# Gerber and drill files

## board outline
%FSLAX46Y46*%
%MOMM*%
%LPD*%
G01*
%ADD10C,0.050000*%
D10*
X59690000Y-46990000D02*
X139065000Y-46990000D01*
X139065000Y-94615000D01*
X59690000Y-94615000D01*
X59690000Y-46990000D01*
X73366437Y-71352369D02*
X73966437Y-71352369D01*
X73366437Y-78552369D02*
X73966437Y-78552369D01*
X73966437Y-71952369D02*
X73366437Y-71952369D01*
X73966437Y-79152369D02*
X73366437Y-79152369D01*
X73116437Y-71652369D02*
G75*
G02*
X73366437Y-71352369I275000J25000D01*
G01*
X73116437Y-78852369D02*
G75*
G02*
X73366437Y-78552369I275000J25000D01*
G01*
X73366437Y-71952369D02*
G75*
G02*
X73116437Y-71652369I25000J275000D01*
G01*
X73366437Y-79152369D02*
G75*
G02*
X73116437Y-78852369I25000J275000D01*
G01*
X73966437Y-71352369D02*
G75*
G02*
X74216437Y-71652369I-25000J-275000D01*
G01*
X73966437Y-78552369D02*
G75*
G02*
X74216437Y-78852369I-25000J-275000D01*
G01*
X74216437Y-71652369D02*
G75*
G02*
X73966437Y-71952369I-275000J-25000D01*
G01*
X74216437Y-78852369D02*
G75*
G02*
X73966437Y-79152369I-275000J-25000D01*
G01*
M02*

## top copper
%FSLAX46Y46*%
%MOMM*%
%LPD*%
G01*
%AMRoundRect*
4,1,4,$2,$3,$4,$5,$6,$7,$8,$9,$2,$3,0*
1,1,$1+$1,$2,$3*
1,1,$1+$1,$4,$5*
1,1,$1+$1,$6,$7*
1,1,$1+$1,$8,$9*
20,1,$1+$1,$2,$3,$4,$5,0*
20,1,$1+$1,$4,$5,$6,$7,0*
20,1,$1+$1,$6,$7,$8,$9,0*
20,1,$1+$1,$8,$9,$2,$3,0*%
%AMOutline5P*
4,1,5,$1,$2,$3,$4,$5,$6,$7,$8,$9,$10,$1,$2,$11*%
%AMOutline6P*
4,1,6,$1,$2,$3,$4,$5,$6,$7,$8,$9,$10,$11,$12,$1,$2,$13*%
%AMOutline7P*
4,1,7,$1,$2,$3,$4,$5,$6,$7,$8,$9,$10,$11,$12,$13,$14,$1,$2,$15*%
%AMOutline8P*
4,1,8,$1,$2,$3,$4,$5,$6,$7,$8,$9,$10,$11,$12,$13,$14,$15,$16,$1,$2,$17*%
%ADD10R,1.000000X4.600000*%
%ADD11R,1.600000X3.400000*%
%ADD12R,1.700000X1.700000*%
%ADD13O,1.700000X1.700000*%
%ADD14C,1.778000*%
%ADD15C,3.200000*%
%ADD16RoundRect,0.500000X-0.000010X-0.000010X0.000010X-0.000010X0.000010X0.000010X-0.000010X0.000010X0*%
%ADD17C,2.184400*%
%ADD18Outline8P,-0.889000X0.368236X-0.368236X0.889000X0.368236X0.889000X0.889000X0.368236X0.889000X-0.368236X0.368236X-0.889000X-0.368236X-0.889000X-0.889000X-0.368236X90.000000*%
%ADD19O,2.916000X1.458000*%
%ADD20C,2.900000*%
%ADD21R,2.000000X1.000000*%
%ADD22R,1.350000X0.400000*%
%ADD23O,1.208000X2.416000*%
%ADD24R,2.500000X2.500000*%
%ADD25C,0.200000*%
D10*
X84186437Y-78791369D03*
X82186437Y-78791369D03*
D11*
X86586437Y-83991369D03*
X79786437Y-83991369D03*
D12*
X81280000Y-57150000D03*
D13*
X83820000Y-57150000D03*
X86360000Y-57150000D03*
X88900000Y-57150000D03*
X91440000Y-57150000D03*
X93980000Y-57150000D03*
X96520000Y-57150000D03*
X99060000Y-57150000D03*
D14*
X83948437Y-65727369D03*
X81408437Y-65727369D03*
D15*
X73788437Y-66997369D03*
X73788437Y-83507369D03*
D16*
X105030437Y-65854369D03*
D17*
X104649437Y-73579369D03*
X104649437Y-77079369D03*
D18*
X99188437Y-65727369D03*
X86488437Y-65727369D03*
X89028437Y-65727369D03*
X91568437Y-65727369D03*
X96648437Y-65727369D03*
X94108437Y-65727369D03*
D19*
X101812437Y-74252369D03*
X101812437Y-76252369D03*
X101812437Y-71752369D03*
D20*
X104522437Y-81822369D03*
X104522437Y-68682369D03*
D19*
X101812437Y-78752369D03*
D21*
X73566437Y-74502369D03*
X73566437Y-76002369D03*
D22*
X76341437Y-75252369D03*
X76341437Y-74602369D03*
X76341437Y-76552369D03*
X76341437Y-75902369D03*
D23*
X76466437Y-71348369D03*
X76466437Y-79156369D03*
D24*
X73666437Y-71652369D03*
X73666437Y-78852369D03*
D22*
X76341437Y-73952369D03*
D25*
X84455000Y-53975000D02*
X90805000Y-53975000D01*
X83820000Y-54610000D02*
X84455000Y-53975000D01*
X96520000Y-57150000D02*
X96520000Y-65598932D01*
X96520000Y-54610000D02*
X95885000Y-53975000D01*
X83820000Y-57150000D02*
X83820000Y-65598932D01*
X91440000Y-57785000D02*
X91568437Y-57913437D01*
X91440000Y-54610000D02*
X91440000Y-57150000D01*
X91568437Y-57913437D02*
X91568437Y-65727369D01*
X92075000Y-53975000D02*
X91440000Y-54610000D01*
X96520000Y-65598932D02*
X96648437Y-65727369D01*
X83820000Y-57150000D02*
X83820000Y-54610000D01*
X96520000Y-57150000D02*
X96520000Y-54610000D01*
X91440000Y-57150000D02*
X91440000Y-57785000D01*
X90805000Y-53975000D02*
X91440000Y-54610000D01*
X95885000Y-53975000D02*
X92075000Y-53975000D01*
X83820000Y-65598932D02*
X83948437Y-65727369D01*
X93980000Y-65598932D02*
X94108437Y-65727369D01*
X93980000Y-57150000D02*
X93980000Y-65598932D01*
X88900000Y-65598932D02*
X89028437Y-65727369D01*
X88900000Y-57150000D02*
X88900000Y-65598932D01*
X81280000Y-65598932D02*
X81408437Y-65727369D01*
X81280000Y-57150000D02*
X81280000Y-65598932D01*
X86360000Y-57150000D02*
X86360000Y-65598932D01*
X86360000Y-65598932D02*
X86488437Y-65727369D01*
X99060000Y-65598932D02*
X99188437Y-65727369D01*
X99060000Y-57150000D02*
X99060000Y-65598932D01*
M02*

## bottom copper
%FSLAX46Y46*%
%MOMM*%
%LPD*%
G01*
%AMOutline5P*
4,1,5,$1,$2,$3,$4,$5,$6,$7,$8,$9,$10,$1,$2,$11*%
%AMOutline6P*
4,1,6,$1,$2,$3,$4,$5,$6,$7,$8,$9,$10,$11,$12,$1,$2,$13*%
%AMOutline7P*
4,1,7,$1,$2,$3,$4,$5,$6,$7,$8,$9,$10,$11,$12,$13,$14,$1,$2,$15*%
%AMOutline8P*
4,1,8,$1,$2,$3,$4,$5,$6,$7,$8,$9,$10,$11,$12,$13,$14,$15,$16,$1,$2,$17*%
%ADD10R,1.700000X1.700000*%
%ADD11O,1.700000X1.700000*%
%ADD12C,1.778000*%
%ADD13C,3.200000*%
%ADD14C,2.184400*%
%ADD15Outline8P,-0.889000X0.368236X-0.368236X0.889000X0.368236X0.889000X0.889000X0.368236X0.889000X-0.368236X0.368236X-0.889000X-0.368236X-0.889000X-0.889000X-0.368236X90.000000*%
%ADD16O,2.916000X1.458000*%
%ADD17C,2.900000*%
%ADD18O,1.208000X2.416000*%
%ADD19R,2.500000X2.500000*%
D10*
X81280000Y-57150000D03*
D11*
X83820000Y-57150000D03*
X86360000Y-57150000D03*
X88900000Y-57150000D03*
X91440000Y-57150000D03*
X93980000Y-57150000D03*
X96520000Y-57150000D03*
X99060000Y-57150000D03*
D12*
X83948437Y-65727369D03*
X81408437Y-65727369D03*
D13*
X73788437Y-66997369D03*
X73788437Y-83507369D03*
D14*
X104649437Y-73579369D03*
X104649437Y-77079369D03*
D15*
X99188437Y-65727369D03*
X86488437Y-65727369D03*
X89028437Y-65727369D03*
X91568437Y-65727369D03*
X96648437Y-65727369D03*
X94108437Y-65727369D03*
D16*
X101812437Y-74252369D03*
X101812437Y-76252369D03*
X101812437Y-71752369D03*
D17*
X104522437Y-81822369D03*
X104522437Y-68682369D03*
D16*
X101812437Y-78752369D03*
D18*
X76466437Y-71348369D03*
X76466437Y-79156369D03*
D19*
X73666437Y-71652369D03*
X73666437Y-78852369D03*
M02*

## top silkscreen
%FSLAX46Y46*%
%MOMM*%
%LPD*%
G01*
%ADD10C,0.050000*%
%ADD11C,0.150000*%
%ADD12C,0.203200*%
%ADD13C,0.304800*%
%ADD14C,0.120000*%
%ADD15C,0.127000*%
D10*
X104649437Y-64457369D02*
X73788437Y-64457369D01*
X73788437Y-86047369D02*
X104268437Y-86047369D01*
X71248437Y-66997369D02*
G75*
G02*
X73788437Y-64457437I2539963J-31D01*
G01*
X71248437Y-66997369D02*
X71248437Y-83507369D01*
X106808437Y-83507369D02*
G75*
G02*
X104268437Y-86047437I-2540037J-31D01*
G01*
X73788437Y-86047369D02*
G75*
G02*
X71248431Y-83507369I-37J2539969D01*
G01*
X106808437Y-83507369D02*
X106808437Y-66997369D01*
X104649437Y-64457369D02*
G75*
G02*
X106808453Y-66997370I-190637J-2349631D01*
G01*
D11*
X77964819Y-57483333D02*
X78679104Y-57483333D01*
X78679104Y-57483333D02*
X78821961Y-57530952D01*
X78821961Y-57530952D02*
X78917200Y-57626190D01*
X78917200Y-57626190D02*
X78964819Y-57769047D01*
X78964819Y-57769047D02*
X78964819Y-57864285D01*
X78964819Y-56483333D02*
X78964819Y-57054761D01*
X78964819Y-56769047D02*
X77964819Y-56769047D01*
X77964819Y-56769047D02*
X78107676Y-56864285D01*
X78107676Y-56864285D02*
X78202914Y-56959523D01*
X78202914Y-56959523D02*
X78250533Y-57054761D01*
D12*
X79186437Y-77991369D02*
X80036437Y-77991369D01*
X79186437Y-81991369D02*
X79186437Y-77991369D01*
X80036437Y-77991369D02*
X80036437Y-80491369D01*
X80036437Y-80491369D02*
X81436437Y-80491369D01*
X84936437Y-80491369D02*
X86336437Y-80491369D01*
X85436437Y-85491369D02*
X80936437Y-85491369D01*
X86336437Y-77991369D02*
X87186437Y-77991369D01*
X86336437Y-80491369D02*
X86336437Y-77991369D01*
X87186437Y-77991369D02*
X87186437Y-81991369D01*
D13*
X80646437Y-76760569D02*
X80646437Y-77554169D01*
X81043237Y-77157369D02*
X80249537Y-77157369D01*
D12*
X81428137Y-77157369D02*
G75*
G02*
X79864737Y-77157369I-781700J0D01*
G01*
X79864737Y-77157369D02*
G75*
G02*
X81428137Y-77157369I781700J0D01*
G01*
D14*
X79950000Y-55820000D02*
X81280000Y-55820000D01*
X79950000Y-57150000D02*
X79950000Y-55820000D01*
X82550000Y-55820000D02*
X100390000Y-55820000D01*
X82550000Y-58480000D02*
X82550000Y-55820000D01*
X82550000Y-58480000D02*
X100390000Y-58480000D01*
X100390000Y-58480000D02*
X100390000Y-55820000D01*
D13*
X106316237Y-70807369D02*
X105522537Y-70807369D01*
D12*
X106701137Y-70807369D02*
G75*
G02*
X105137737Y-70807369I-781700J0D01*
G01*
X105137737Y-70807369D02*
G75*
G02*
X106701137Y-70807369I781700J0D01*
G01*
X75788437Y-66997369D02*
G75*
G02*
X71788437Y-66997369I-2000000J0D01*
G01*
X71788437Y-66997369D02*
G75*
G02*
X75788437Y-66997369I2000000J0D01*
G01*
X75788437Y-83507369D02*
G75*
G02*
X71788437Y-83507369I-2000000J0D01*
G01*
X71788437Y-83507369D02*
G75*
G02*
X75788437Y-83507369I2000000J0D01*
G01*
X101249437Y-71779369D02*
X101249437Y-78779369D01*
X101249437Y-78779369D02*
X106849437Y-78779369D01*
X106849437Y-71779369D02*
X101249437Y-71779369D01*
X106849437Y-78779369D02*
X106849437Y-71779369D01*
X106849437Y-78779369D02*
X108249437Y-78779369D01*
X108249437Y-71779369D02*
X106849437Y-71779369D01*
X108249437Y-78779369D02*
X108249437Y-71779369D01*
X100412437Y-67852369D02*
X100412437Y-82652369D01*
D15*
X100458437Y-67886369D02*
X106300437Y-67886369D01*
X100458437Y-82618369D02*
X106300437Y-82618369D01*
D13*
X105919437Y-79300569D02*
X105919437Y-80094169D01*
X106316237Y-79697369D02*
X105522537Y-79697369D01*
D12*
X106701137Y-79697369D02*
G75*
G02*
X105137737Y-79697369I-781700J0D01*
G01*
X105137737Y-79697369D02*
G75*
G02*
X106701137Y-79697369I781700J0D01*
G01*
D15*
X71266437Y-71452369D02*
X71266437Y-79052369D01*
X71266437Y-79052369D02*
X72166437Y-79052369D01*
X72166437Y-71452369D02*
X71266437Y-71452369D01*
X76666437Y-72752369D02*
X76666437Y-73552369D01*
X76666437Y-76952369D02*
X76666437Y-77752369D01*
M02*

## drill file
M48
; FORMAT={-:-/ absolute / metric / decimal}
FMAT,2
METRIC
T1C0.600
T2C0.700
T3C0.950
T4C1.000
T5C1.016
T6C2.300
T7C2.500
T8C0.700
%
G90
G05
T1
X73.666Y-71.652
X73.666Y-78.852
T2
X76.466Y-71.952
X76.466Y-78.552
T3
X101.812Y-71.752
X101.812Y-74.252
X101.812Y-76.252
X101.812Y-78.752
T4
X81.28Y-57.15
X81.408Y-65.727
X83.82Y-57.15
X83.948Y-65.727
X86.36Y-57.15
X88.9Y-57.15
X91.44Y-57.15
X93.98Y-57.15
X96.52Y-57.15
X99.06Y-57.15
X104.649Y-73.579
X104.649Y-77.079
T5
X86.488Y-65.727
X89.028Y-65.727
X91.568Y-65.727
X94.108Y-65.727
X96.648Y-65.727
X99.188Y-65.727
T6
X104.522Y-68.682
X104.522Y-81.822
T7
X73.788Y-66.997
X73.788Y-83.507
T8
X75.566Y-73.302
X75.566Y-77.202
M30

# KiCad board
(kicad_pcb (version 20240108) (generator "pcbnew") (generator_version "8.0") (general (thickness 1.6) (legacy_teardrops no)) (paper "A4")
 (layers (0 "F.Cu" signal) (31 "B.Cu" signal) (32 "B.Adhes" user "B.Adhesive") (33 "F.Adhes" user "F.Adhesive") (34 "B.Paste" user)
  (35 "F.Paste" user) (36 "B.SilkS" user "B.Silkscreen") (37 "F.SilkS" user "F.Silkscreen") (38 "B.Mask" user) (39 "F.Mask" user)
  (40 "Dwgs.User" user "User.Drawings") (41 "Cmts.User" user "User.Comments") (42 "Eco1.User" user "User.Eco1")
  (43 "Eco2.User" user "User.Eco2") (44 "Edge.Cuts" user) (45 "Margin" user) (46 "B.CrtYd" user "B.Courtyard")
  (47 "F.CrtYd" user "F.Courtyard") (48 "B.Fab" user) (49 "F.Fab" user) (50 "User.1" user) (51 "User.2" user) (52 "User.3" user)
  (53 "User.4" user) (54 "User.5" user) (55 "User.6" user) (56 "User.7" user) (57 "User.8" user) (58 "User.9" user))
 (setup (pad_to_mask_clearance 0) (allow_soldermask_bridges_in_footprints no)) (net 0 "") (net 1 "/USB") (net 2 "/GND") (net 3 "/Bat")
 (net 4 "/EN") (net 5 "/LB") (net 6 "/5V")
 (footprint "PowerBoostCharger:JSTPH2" (layer "F.Cu") (at 83.186437 82.491369 180)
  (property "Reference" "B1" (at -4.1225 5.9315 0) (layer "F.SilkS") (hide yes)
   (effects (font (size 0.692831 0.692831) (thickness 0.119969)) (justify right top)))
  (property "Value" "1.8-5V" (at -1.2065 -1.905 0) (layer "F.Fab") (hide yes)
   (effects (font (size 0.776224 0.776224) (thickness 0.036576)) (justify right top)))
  (fp_line (start 4 4.5) (end 3.15 4.5) (stroke (width 0.2032) (type solid)) (layer "F.SilkS"))
  (fp_line (start 4 0.5) (end 4 4.5) (stroke (width 0.2032) (type solid)) (layer "F.SilkS"))
  (fp_line (start 3.15 4.5) (end 3.15 2) (stroke (width 0.2032) (type solid)) (layer "F.SilkS"))
  (fp_line (start 3.15 2) (end 1.75 2) (stroke (width 0.2032) (type solid)) (layer "F.SilkS"))
  (fp_line (start -1.75 2) (end -3.15 2) (stroke (width 0.2032) (type solid)) (layer "F.SilkS"))
  (fp_line (start -2.25 -3) (end 2.25 -3) (stroke (width 0.2032) (type solid)) (layer "F.SilkS"))
  (fp_line (start -3.15 4.5) (end -4 4.5) (stroke (width 0.2032) (type solid)) (layer "F.SilkS"))
  (fp_line (start -3.15 2) (end -3.15 4.5) (stroke (width 0.2032) (type solid)) (layer "F.SilkS"))
  (fp_line (start -4 4.5) (end -4 0.5) (stroke (width 0.2032) (type solid)) (layer "F.SilkS"))
  (pad "1" smd rect (at -1 3.7 180) (size 1 4.6) (layers "F.Cu" "F.Paste" "F.Mask") (solder_mask_margin 0.0508) (thermal_bridge_angle 45))
  (pad "2" smd rect (at 1 3.7 180) (size 1 4.6) (layers "F.Cu" "F.Paste" "F.Mask") (solder_mask_margin 0.0508) (thermal_bridge_angle 45))
  (pad "NC1" smd rect (at -3.4 -1.5 270) (size 3.4 1.6) (layers "F.Cu" "F.Paste" "F.Mask") (solder_mask_margin 0.0508)
   (thermal_bridge_angle 45))
  (pad "NC2" smd rect (at 3.4 -1.5 270) (size 3.4 1.6) (layers "F.Cu" "F.Paste" "F.Mask") (solder_mask_margin 0.0508)
   (thermal_bridge_angle 45)))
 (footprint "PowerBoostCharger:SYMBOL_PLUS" (layer "F.Cu") (at 80.646437 77.157369)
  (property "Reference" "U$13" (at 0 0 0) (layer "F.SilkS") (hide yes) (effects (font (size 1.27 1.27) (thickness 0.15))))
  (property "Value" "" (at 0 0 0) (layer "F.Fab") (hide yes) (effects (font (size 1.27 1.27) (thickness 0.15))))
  (fp_line (start 0 -0.3968) (end 0 0.3968) (stroke (width 0.3048) (type solid)) (layer "F.SilkS"))
  (fp_line (start 0.3968 0) (end -0.3969 0) (stroke (width 0.3048) (type solid)) (layer "F.SilkS"))
  (fp_circle (center 0 0) (end 0.7817 0) (stroke (width 0.2032) (type solid)) (fill none) (layer "F.SilkS")))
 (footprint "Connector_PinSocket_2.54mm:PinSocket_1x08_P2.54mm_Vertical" (layer "F.Cu") (at 81.28 57.15 90)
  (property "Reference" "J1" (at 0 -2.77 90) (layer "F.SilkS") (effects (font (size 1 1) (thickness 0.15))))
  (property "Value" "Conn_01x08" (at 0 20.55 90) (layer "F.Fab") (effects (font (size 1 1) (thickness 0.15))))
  (fp_line (start 1.33 -1.33) (end 1.33 0) (stroke (width 0.12) (type solid)) (layer "F.SilkS"))
  (fp_line (start 0 -1.33) (end 1.33 -1.33) (stroke (width 0.12) (type solid)) (layer "F.SilkS"))
  (fp_line (start 1.33 1.27) (end 1.33 19.11) (stroke (width 0.12) (type solid)) (layer "F.SilkS"))
  (fp_line (start -1.33 1.27) (end 1.33 1.27) (stroke (width 0.12) (type solid)) (layer "F.SilkS"))
  (fp_line (start -1.33 1.27) (end -1.33 19.11) (stroke (width 0.12) (type solid)) (layer "F.SilkS"))
  (fp_line (start -1.33 19.11) (end 1.33 19.11) (stroke (width 0.12) (type solid)) (layer "F.SilkS"))
  (pad "1" thru_hole rect (at 0 0 90) (size 1.7 1.7) (drill 1) (layers "*.Cu" "*.Mask") (remove_unused_layers no) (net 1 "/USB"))
  (pad "2" thru_hole oval (at 0 2.54 90) (size 1.7 1.7) (drill 1) (layers "*.Cu" "*.Mask") (remove_unused_layers no) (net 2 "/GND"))
  (pad "3" thru_hole oval (at 0 5.08 90) (size 1.7 1.7) (drill 1) (layers "*.Cu" "*.Mask") (remove_unused_layers no) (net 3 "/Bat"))
  (pad "4" thru_hole oval (at 0 7.62 90) (size 1.7 1.7) (drill 1) (layers "*.Cu" "*.Mask") (remove_unused_layers no) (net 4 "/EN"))
  (pad "5" thru_hole oval (at 0 10.16 90) (size 1.7 1.7) (drill 1) (layers "*.Cu" "*.Mask") (remove_unused_layers no) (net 2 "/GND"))
  (pad "6" thru_hole oval (at 0 12.7 90) (size 1.7 1.7) (drill 1) (layers "*.Cu" "*.Mask") (remove_unused_layers no) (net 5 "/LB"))
  (pad "7" thru_hole oval (at 0 15.24 90) (size 1.7 1.7) (drill 1) (layers "*.Cu" "*.Mask") (remove_unused_layers no) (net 2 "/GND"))
  (pad "8" thru_hole oval (at 0 17.78 90) (size 1.7 1.7) (drill 1) (layers "*.Cu" "*.Mask") (remove_unused_layers no) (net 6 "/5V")))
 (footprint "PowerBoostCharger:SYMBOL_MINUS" (layer "F.Cu") (at 105.919437 70.807369)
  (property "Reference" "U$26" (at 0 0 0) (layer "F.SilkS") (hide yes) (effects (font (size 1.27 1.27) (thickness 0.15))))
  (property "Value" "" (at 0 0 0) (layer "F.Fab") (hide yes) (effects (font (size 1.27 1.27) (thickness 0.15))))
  (fp_line (start 0.3968 0) (end -0.3969 0) (stroke (width 0.3048) (type solid)) (layer "F.SilkS"))
  (fp_circle (center 0 0) (end 0.7817 0) (stroke (width 0.2032) (type solid)) (fill none) (layer "F.SilkS")))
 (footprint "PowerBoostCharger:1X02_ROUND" (layer "F.Cu") (at 82.678437 65.727369)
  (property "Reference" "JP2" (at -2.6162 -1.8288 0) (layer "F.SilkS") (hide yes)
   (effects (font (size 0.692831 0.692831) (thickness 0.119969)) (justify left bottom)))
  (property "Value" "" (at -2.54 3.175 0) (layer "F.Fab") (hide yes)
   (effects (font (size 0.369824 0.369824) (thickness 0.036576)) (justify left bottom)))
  (pad "GND" thru_hole circle (at 1.27 0 90) (size 1.778 1.778) (drill 1) (layers "*.Cu" "*.Mask") (remove_unused_layers no) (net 2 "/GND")
   (solder_mask_margin 0.0508))
  (pad "USB" thru_hole circle (at -1.27 0 90) (size 1.778 1.778) (drill 1) (layers "*.Cu" "*.Mask") (remove_unused_layers no) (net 1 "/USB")
   (solder_mask_margin 0.0508)))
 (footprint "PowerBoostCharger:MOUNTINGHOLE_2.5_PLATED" (layer "F.Cu") (at 73.788437 66.997369)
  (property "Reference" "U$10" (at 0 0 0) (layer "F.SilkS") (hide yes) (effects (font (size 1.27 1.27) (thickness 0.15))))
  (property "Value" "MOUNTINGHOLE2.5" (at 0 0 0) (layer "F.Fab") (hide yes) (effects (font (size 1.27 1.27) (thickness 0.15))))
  (fp_circle (center 0 0) (end 2 0) (stroke (width 0.2032) (type solid)) (fill none) (layer "F.SilkS"))
  (pad "P$1" thru_hole circle (at 0 0) (size 3.2 3.2) (drill 2.5) (layers "*.Cu" "*.Mask") (remove_unused_layers no)
   (solder_mask_margin 0.0508))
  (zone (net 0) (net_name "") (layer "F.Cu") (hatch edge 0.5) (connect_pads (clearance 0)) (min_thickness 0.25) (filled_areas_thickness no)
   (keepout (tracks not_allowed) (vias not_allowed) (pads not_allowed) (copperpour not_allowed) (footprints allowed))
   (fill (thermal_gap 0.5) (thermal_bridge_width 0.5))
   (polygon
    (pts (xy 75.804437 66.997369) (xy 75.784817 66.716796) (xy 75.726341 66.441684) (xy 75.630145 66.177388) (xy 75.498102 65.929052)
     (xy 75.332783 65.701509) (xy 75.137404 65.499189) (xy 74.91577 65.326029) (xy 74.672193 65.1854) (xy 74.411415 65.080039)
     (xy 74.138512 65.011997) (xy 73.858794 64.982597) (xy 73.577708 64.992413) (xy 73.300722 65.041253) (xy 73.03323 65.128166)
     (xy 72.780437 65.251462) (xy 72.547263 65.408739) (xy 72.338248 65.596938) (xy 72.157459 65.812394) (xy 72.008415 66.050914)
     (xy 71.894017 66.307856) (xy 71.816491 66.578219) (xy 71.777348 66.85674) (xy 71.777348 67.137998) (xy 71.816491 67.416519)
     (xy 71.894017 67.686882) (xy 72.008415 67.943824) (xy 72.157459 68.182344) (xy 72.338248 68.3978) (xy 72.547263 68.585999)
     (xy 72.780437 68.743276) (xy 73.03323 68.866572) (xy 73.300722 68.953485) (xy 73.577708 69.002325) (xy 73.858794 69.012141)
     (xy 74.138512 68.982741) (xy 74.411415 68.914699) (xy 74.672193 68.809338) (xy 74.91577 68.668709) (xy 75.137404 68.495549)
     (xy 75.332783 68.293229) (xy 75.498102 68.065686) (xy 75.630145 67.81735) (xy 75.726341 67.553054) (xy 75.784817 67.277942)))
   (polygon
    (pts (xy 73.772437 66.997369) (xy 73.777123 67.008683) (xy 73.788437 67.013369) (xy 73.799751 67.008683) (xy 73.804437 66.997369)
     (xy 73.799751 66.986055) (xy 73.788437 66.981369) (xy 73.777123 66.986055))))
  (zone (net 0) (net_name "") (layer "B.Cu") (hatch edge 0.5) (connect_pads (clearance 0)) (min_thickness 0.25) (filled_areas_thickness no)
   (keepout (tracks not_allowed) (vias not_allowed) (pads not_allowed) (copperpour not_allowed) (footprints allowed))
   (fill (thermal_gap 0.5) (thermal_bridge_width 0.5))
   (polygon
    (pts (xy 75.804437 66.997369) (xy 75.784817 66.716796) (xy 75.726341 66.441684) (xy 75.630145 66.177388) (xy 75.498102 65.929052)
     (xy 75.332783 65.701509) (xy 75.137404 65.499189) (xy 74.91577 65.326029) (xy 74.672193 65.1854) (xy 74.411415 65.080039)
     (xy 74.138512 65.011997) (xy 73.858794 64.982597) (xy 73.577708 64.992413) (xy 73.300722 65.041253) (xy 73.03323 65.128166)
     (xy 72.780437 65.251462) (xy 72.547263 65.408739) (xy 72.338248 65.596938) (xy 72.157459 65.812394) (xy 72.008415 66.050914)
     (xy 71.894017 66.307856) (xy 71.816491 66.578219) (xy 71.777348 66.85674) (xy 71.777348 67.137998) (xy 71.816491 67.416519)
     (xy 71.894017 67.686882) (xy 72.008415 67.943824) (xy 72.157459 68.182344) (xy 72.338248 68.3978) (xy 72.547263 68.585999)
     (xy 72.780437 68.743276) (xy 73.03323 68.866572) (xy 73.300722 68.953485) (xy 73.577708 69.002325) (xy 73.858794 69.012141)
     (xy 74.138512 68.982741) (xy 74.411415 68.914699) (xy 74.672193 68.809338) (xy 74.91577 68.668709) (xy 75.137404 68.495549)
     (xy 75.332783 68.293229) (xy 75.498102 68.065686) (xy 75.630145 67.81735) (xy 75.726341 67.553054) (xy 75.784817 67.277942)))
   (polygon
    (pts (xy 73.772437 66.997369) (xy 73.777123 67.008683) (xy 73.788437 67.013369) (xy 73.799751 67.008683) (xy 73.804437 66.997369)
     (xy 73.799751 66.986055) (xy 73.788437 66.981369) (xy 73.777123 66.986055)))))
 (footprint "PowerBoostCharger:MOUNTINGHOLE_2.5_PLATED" (layer "F.Cu") (at 73.788437 83.507369)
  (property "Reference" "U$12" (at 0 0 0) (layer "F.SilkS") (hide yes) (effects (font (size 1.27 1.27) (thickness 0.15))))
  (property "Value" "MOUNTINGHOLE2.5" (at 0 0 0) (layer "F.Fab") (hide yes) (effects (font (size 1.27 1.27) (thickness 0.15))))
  (fp_circle (center 0 0) (end 2 0) (stroke (width 0.2032) (type solid)) (fill none) (layer "F.SilkS"))
  (pad "P$1" thru_hole circle (at 0 0) (size 3.2 3.2) (drill 2.5) (layers "*.Cu" "*.Mask") (remove_unused_layers no)
   (solder_mask_margin 0.0508))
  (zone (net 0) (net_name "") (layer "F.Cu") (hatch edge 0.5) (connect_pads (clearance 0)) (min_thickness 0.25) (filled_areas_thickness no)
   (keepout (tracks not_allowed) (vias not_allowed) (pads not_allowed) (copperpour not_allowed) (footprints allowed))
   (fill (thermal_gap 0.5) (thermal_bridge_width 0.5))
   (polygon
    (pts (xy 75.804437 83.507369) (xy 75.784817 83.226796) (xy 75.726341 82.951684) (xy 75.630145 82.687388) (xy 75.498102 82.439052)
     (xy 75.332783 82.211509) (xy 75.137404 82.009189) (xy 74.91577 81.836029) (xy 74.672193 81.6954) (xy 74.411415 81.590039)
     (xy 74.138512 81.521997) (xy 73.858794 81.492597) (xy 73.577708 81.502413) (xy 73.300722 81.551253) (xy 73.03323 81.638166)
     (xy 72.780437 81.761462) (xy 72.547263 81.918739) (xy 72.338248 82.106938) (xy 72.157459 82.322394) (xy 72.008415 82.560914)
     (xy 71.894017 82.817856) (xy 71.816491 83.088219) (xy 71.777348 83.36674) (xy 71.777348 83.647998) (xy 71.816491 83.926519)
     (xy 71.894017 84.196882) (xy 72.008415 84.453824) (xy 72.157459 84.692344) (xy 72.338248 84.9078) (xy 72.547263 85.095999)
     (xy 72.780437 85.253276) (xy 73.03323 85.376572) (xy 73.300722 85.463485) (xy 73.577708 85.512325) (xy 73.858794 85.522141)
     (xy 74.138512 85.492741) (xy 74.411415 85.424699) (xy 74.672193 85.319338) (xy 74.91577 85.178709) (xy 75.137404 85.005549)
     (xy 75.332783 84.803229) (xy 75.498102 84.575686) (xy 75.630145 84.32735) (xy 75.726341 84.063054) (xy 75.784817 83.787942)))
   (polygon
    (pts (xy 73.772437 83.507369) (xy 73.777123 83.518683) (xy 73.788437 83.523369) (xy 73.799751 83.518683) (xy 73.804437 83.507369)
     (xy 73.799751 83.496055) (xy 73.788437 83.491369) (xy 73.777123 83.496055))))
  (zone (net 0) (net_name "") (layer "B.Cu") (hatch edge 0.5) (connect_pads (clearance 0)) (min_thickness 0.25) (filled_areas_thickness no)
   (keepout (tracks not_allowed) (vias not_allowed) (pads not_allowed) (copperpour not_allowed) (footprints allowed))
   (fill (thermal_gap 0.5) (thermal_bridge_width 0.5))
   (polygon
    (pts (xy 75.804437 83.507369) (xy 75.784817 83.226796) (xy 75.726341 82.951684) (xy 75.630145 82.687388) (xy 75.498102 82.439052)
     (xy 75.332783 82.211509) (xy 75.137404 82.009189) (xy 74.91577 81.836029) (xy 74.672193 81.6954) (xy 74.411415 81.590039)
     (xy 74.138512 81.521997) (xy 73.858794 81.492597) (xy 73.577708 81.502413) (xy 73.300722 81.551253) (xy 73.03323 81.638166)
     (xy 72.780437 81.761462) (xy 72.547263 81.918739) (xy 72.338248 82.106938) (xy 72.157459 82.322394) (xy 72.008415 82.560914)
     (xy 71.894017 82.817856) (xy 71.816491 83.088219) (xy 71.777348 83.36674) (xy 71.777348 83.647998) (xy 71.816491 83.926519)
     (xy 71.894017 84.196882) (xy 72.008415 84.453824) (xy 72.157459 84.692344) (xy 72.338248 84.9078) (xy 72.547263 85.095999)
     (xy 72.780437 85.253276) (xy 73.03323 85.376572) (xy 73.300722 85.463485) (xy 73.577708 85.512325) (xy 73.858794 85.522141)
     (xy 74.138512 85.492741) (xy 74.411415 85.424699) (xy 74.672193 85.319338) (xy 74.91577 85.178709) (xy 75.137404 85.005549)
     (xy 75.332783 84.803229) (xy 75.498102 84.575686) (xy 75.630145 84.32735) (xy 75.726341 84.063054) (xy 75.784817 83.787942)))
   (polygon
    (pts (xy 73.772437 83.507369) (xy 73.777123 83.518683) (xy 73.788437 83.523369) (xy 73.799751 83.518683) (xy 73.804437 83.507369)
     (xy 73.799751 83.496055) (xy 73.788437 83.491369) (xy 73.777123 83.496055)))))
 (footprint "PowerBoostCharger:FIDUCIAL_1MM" (layer "F.Cu") (at 105.030437 65.854369)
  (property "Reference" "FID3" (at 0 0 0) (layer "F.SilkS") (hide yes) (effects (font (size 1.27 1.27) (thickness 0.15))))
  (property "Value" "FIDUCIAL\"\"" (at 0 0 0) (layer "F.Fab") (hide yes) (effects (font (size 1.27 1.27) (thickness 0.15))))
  (pad "1" smd roundrect (at 0 0) (size 1 1) (layers "F.Cu" "F.Mask") (roundrect_rratio 0.5) (solder_mask_margin 0.0508)
   (thermal_bridge_angle 45)))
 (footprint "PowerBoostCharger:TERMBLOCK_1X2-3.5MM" (layer "F.Cu") (at 104.649437 75.379369 90)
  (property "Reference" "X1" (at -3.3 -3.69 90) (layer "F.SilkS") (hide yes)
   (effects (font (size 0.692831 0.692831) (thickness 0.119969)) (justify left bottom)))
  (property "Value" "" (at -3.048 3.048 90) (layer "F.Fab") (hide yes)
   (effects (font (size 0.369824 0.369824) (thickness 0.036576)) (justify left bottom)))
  (fp_line (start 3.6 -3.4) (end -3.4 -3.4) (stroke (width 0.2032) (type solid)) (layer "F.SilkS"))
  (fp_line (start -3.4 -3.4) (end -3.4 2.2) (stroke (width 0.2032) (type solid)) (layer "F.SilkS"))
  (fp_line (start 3.6 2.2) (end 3.6 -3.4) (stroke (width 0.2032) (type solid)) (layer "F.SilkS"))
  (fp_line (start -3.4 2.2) (end 3.6 2.2) (stroke (width 0.2032) (type solid)) (layer "F.SilkS"))
  (fp_line (start -3.4 2.2) (end -3.4 3.6) (stroke (width 0.2032) (type solid)) (layer "F.SilkS"))
  (fp_line (start 3.6 3.6) (end 3.6 2.2) (stroke (width 0.2032) (type solid)) (layer "F.SilkS"))
  (fp_line (start -3.4 3.6) (end 3.6 3.6) (stroke (width 0.2032) (type solid)) (layer "F.SilkS"))
  (pad "1" thru_hole circle (at 1.8 0 90) (size 2.1844 2.1844) (drill 1) (layers "*.Cu" "*.Mask") (remove_unused_layers no)
   (solder_mask_margin 0.0508))
  (pad "2" thru_hole circle (at -1.7 0 90) (size 2.1844 2.1844) (drill 1) (layers "*.Cu" "*.Mask") (remove_unused_layers no)
   (solder_mask_margin 0.0508)))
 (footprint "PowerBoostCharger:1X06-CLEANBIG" (layer "F.Cu") (at 92.838437 65.727369)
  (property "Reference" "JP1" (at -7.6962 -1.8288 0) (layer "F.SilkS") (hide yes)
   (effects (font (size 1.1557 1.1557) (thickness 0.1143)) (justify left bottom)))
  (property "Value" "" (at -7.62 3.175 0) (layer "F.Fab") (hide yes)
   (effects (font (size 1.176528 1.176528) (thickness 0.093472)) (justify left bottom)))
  (pad "5V" thru_hole roundrect (at 6.35 0 90) (size 1.778 1.778) (drill 1.016) (layers "*.Cu" "*.Mask") (remove_unused_layers no)
   (roundrect_rratio 0.25) (chamfer_ratio 0.2928932188) (chamfer top_left top_right bottom_left bottom_right) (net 6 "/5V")
   (solder_mask_margin 0.0508) (thermal_bridge_angle 45))
  (pad "Bat" thru_hole roundrect (at -6.35 0 90) (size 1.778 1.778) (drill 1.016) (layers "*.Cu" "*.Mask") (remove_unused_layers no)
   (roundrect_rratio 0.25) (chamfer_ratio 0.2928932188) (chamfer top_left top_right bottom_left bottom_right) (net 3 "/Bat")
   (solder_mask_margin 0.0508) (thermal_bridge_angle 45))
  (pad "EN" thru_hole roundrect (at -3.81 0 90) (size 1.778 1.778) (drill 1.016) (layers "*.Cu" "*.Mask") (remove_unused_layers no)
   (roundrect_rratio 0.25) (chamfer_ratio 0.2928932188) (chamfer top_left top_right bottom_left bottom_right) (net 4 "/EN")
   (solder_mask_margin 0.0508) (thermal_bridge_angle 45))
  (pad "GND" thru_hole roundrect (at -1.27 0 90) (size 1.778 1.778) (drill 1.016) (layers "*.Cu" "*.Mask") (remove_unused_layers no)
   (roundrect_rratio 0.25) (chamfer_ratio 0.2928932188) (chamfer top_left top_right bottom_left bottom_right) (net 2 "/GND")
   (solder_mask_margin 0.0508) (thermal_bridge_angle 45))
  (pad "GND" thru_hole roundrect (at 3.81 0 90) (size 1.778 1.778) (drill 1.016) (layers "*.Cu" "*.Mask") (remove_unused_layers no)
   (roundrect_rratio 0.25) (chamfer_ratio 0.2928932188) (chamfer top_left top_right bottom_left bottom_right) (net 2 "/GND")
   (solder_mask_margin 0.0508) (thermal_bridge_angle 45))
  (pad "LB" thru_hole roundrect (at 1.27 0 90) (size 1.778 1.778) (drill 1.016) (layers "*.Cu" "*.Mask") (remove_unused_layers no)
   (roundrect_rratio 0.25) (chamfer_ratio 0.2928932188) (chamfer top_left top_right bottom_left bottom_right) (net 5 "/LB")
   (solder_mask_margin 0.0508) (thermal_bridge_angle 45)))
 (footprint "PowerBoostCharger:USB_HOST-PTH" (layer "F.Cu") (at 108.332437 75.252369 90)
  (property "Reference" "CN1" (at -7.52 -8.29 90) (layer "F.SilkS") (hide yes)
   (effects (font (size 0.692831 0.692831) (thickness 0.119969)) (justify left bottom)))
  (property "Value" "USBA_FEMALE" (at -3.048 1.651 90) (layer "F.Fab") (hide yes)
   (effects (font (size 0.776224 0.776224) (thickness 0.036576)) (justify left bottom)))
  (fp_line (start 7.4 -7.92) (end -7.4 -7.92) (stroke (width 0.2032) (type solid)) (layer "F.SilkS"))
  (fp_line (start 7.366 -7.874) (end 7.366 -2.032) (stroke (width 0.127) (type solid)) (layer "F.SilkS"))
  (fp_line (start -7.366 -7.874) (end -7.366 -2.032) (stroke (width 0.127) (type solid)) (layer "F.SilkS"))
  (pad "D+" thru_hole oval (at 1 -6.52 180) (size 2.916 1.458) (drill 0.95) (layers "*.Cu" "*.Mask") (remove_unused_layers no)
   (solder_mask_margin 0.0508) (thermal_bridge_angle 45))
  (pad "D-" thru_hole oval (at -1 -6.52 180) (size 2.916 1.458) (drill 0.95) (layers "*.Cu" "*.Mask") (remove_unused_layers no)
   (solder_mask_margin 0.0508) (thermal_bridge_angle 45))
  (pad "GND" thru_hole oval (at 3.5 -6.52 180) (size 2.916 1.458) (drill 0.95) (layers "*.Cu" "*.Mask") (remove_unused_layers no)
   (solder_mask_margin 0.0508) (thermal_bridge_angle 45))
  (pad "S1" thru_hole circle (at -6.57 -3.81 90) (size 2.9 2.9) (drill 2.3) (layers "*.Cu" "*.Mask") (remove_unused_layers no)
   (solder_mask_margin 0.0508))
  (pad "S2" thru_hole circle (at 6.57 -3.81 270) (size 2.9 2.9) (drill 2.3) (layers "*.Cu" "*.Mask") (remove_unused_layers no)
   (solder_mask_margin 0.0508))
  (pad "VBUS" thru_hole oval (at -3.5 -6.52 180) (size 2.916 1.458) (drill 0.95) (layers "*.Cu" "*.Mask") (remove_unused_layers no)
   (solder_mask_margin 0.0508) (thermal_bridge_angle 45)))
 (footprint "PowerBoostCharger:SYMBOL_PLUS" (layer "F.Cu") (at 105.919437 79.697369)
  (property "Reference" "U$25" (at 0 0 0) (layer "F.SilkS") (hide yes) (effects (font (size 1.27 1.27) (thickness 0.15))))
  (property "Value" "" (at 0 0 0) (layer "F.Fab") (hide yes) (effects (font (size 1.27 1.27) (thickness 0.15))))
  (fp_line (start 0 -0.3968) (end 0 0.3968) (stroke (width 0.3048) (type solid)) (layer "F.SilkS"))
  (fp_line (start 0.3968 0) (end -0.3969 0) (stroke (width 0.3048) (type solid)) (layer "F.SilkS"))
  (fp_circle (center 0 0) (end 0.7817 0) (stroke (width 0.2032) (type solid)) (fill none) (layer "F.SilkS")))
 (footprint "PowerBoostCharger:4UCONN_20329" (layer "F.Cu") (at 75.566437 75.252369 -90)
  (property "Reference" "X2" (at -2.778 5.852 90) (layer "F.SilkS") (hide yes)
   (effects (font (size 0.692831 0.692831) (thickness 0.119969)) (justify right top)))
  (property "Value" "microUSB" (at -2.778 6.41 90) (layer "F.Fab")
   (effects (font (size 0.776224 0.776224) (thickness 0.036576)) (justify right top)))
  (fp_line (start -3.8 4.3) (end 3.8 4.3) (stroke (width 0.127) (type solid)) (layer "F.SilkS"))
  (fp_line (start 3.8 4.3) (end 3.8 3.4) (stroke (width 0.127) (type solid)) (layer "F.SilkS"))
  (fp_line (start -3.8 3.4) (end -3.8 4.3) (stroke (width 0.127) (type solid)) (layer "F.SilkS"))
  (fp_line (start -2.5 -1.1) (end -1.7 -1.1) (stroke (width 0.127) (type solid)) (layer "F.SilkS"))
  (fp_line (start 1.7 -1.1) (end 2.5 -1.1) (stroke (width 0.127) (type solid)) (layer "F.SilkS"))
  (fp_line (start -3.9 2.2) (end -3.9 1.6) (stroke (width 0.05) (type solid)) (layer "Edge.Cuts"))
  (fp_line (start 3.3 2.2) (end 3.3 1.6) (stroke (width 0.05) (type solid)) (layer "Edge.Cuts"))
  (fp_line (start -3.3 1.6) (end -3.3 2.2) (stroke (width 0.05) (type solid)) (layer "Edge.Cuts"))
  (fp_line (start 3.9 1.6) (end 3.9 2.2) (stroke (width 0.05) (type solid)) (layer "Edge.Cuts"))
  (fp_arc (start -3.6 2.45) (mid -3.801777 2.387132) (end -3.9 2.2) (stroke (width 0.05) (type solid)) (layer "Edge.Cuts"))
  (fp_arc (start 3.6 2.45) (mid 3.398223 2.387132) (end 3.3 2.2) (stroke (width 0.05) (type solid)) (layer "Edge.Cuts"))
  (fp_arc (start -3.3 2.2) (mid -3.398223 2.387132) (end -3.6 2.45) (stroke (width 0.05) (type solid)) (layer "Edge.Cuts"))
  (fp_arc (start 3.9 2.2) (mid 3.801777 2.387132) (end 3.6 2.45) (stroke (width 0.05) (type solid)) (layer "Edge.Cuts"))
  (fp_arc (start -3.9 1.6) (mid -3.801777 1.412868) (end -3.6 1.35) (stroke (width 0.05) (type solid)) (layer "Edge.Cuts"))
  (fp_arc (start 3.3 1.6) (mid 3.398223 1.412868) (end 3.6 1.35) (stroke (width 0.05) (type solid)) (layer "Edge.Cuts"))
  (fp_arc (start -3.6 1.35) (mid -3.398223 1.412868) (end -3.3 1.6) (stroke (width 0.05) (type solid)) (layer "Edge.Cuts"))
  (fp_arc (start 3.6 1.35) (mid 3.801777 1.412868) (end 3.9 1.6) (stroke (width 0.05) (type solid)) (layer "Edge.Cuts"))
  (pad "" np_thru_hole circle (at -1.95 0 270) (size 0.7 0.7) (drill 0.7) (layers "F&B.Cu" "*.Mask"))
  (pad "" np_thru_hole circle (at 1.95 0 270) (size 0.7 0.7) (drill 0.7) (layers "F&B.Cu" "*.Mask"))
  (pad "BASE@1" smd rect (at -0.75 2) (size 2 1) (layers "F.Cu" "F.Paste" "F.Mask") (solder_mask_margin 0.0508) (thermal_bridge_angle 45))
  (pad "BASE@2" smd rect (at 0.75 2) (size 2 1) (layers "F.Cu" "F.Paste" "F.Mask") (solder_mask_margin 0.0508) (thermal_bridge_angle 45))
  (pad "D+" smd rect (at 0 -0.775 270) (size 0.4 1.35) (layers "F.Cu" "F.Paste") (solder_mask_margin 0.0508) (thermal_bridge_angle 45))
  (pad "D-" smd rect (at -0.65 -0.775 270) (size 0.4 1.35) (layers "F.Cu" "F.Paste") (solder_mask_margin 0.0508) (thermal_bridge_angle 45))
  (pad "GND" smd rect (at 1.3 -0.775 270) (size 0.4 1.35) (layers "F.Cu" "F.Paste") (solder_mask_margin 0.0508) (thermal_bridge_angle 45))
  (pad "ID" smd rect (at 0.65 -0.775 270) (size 0.4 1.35) (layers "F.Cu" "F.Paste") (solder_mask_margin 0.0508) (thermal_bridge_angle 45))
  (pad "SPRT@1" thru_hole oval (at -3.3 -0.9 90) (size 2.416 1.208) (drill 0.7 (offset 0.604 0)) (layers "*.Cu" "*.Mask")
   (remove_unused_layers no) (solder_mask_margin 0.0508) (thermal_bridge_angle 45))
  (pad "SPRT@2" thru_hole oval (at 3.3 -0.9 270) (size 2.416 1.208) (drill 0.7 (offset 0.604 0)) (layers "*.Cu" "*.Mask")
   (remove_unused_layers no) (solder_mask_margin 0.0508) (thermal_bridge_angle 45))
  (pad "SPRT@3" thru_hole rect (at -3.6 1.9) (size 2.5 2.5) (drill 0.6) (layers "*.Cu" "*.Mask") (remove_unused_layers no)
   (solder_mask_margin 0.0508) (thermal_bridge_angle 45))
  (pad "SPRT@4" thru_hole rect (at 3.6 1.9) (size 2.5 2.5) (drill 0.6) (layers "*.Cu" "*.Mask") (remove_unused_layers no)
   (solder_mask_margin 0.0508) (thermal_bridge_angle 45))
  (pad "VBUS" smd rect (at -1.3 -0.775 270) (size 0.4 1.35) (layers "F.Cu" "F.Paste") (solder_mask_margin 0.0508) (thermal_bridge_angle 45)))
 (gr_line (start 104.649437 64.457369) (end 73.788437 64.457369) (stroke (width 0.05) (type solid)) (layer "F.SilkS"))
 (gr_line (start 73.788437 86.047369) (end 104.268437 86.047369) (stroke (width 0.05) (type solid)) (layer "F.SilkS"))
 (gr_arc (start 71.248437 66.997369) (mid 71.992386 65.201318) (end 73.788437 64.457369) (stroke (width 0.05) (type solid))
  (layer "F.SilkS"))
 (gr_line (start 71.248437 66.997369) (end 71.248437 83.507369) (stroke (width 0.05) (type solid)) (layer "F.SilkS"))
 (gr_arc (start 106.808437 83.507369) (mid 106.064489 85.303421) (end 104.268437 86.047369) (stroke (width 0.05) (type solid))
  (layer "F.SilkS"))
 (gr_arc (start 73.788437 86.047369) (mid 71.992386 85.30342) (end 71.248437 83.507369) (stroke (width 0.05) (type solid)) (layer "F.SilkS"))
 (gr_line (start 106.808437 83.507369) (end 106.808437 66.997369) (stroke (width 0.05) (type solid)) (layer "F.SilkS"))
 (gr_arc (start 104.649437 64.457369) (mid 106.25495 65.280258) (end 106.808437 66.997369) (stroke (width 0.05) (type solid))
  (layer "F.SilkS"))
 (gr_rect (start 59.69 46.99) (end 139.065 94.615) (stroke (width 0.05) (type default)) (fill none) (layer "Edge.Cuts"))
 (segment (start 84.455 53.975) (end 90.805 53.975) (width 0.2) (layer "F.Cu") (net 2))
 (segment (start 83.82 54.61) (end 84.455 53.975) (width 0.2) (layer "F.Cu") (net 2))
 (segment (start 96.52 57.15) (end 96.52 65.598932) (width 0.2) (layer "F.Cu") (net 2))
 (segment (start 96.52 54.61) (end 95.885 53.975) (width 0.2) (layer "F.Cu") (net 2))
 (segment (start 83.82 57.15) (end 83.82 65.598932) (width 0.2) (layer "F.Cu") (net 2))
 (segment (start 91.44 57.785) (end 91.568437 57.913437) (width 0.2) (layer "F.Cu") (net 2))
 (segment (start 91.44 54.61) (end 91.44 57.15) (width 0.2) (layer "F.Cu") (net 2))
 (segment (start 91.568437 57.913437) (end 91.568437 65.727369) (width 0.2) (layer "F.Cu") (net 2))
 (segment (start 92.075 53.975) (end 91.44 54.61) (width 0.2) (layer "F.Cu") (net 2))
 (segment (start 96.52 65.598932) (end 96.648437 65.727369) (width 0.2) (layer "F.Cu") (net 2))
 (segment (start 83.82 57.15) (end 83.82 54.61) (width 0.2) (layer "F.Cu") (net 2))
 (segment (start 96.52 57.15) (end 96.52 54.61) (width 0.2) (layer "F.Cu") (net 2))
 (segment (start 91.44 57.15) (end 91.44 57.785) (width 0.2) (layer "F.Cu") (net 2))
 (segment (start 90.805 53.975) (end 91.44 54.61) (width 0.2) (layer "F.Cu") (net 2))
 (segment (start 95.885 53.975) (end 92.075 53.975) (width 0.2) (layer "F.Cu") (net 2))
 (segment (start 83.82 65.598932) (end 83.948437 65.727369) (width 0.2) (layer "F.Cu") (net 2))
 (segment (start 93.98 65.598932) (end 94.108437 65.727369) (width 0.2) (layer "F.Cu") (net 5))
 (segment (start 93.98 57.15) (end 93.98 65.598932) (width 0.2) (layer "F.Cu") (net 5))
 (segment (start 88.9 65.598932) (end 89.028437 65.727369) (width 0.2) (layer "F.Cu") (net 4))
 (segment (start 88.9 57.15) (end 88.9 65.598932) (width 0.2) (layer "F.Cu") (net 4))
 (segment (start 81.28 65.598932) (end 81.408437 65.727369) (width 0.2) (layer "F.Cu") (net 1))
 (segment (start 81.28 57.15) (end 81.28 65.598932) (width 0.2) (layer "F.Cu") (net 1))
 (segment (start 86.36 57.15) (end 86.36 65.598932) (width 0.2) (layer "F.Cu") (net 3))
 (segment (start 86.36 65.598932) (end 86.488437 65.727369) (width 0.2) (layer "F.Cu") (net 3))
 (segment (start 99.06 65.598932) (end 99.188437 65.727369) (width 0.2) (layer "F.Cu") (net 6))
 (segment (start 99.06 57.15) (end 99.06 65.598932) (width 0.2) (layer "F.Cu") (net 6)))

